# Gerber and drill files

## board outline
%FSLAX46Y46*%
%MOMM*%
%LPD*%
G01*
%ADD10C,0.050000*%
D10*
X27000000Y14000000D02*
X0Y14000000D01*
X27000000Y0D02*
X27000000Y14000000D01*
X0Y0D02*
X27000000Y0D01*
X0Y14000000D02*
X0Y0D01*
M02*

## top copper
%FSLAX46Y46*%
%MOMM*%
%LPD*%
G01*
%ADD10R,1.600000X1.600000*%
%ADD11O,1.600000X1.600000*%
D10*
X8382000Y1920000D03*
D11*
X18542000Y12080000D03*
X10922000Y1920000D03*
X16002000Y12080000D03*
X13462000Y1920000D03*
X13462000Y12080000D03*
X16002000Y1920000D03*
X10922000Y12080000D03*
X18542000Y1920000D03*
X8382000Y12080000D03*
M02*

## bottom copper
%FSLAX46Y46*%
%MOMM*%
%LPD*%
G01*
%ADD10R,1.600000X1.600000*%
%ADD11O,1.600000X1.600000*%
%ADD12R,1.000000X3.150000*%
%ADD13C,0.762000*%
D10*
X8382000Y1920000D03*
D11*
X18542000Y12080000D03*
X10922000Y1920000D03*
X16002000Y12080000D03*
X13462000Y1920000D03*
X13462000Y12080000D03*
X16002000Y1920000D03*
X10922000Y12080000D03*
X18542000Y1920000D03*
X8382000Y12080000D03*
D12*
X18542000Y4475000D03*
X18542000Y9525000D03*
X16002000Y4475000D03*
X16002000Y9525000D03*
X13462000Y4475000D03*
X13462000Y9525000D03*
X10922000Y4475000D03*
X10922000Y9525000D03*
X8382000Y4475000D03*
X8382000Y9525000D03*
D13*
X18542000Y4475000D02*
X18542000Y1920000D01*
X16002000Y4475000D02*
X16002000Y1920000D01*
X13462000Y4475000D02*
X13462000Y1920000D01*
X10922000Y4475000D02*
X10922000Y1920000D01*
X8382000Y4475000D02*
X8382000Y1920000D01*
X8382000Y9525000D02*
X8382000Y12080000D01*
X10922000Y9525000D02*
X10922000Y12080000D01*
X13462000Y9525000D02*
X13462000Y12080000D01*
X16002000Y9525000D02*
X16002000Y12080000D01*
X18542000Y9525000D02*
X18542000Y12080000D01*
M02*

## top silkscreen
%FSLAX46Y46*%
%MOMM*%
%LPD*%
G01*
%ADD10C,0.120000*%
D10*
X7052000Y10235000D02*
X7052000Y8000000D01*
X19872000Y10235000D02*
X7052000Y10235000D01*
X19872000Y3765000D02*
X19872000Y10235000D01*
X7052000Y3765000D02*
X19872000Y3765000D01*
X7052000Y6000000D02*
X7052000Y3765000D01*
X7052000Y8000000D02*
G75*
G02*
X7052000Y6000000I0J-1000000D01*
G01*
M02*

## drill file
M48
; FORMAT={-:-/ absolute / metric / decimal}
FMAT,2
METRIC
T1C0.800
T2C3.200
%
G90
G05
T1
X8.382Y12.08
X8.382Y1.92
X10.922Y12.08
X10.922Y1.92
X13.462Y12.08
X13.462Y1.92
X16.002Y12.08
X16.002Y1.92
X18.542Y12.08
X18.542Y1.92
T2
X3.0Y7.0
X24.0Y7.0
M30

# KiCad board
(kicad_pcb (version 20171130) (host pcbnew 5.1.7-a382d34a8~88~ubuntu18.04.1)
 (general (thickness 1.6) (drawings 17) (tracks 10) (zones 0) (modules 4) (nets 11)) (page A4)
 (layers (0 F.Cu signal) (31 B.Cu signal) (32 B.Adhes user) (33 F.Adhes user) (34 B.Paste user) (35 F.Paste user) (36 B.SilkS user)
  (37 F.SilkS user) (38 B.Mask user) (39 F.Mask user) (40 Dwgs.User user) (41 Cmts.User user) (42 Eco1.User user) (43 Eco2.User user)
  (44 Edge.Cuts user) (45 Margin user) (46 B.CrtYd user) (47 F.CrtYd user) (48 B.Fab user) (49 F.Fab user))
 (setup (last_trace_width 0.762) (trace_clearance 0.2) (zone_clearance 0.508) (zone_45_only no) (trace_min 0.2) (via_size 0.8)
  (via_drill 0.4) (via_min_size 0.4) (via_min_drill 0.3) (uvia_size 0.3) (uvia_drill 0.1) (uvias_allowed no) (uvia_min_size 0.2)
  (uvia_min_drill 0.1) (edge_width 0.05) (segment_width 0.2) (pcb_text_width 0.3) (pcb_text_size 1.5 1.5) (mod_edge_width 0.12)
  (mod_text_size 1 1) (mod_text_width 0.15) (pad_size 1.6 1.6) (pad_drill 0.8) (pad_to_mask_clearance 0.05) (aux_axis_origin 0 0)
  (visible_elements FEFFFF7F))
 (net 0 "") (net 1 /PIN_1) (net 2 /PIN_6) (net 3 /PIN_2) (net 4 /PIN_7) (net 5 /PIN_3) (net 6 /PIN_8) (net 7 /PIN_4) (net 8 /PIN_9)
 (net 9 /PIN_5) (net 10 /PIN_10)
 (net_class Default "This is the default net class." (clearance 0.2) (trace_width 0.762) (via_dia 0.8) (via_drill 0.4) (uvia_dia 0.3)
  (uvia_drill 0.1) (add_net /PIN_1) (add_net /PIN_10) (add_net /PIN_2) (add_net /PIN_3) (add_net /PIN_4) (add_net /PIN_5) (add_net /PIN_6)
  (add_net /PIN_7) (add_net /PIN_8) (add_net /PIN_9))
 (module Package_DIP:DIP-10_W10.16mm (layer F.Cu) (at 8.382 -1.92 90)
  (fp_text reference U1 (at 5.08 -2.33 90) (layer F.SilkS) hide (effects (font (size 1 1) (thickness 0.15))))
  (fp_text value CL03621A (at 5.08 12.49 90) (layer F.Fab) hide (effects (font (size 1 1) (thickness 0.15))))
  (fp_line (start 8.315 -1.33) (end 6.08 -1.33) (layer F.SilkS) (width 0.12))
  (fp_line (start 8.315 11.49) (end 8.315 -1.33) (layer F.SilkS) (width 0.12))
  (fp_line (start 1.845 11.49) (end 8.315 11.49) (layer F.SilkS) (width 0.12))
  (fp_line (start 1.845 -1.33) (end 1.845 11.49) (layer F.SilkS) (width 0.12))
  (fp_line (start 4.08 -1.33) (end 1.845 -1.33) (layer F.SilkS) (width 0.12))
  (fp_arc (start 5.08 -1.33) (end 4.08 -1.33) (angle -180) (layer F.SilkS) (width 0.12))
  (pad 1 thru_hole rect (at 0 0 90) (size 1.6 1.6) (drill 0.8) (layers *.Cu *.Mask) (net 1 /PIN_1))
  (pad 6 thru_hole oval (at 10.16 10.16 90) (size 1.6 1.6) (drill 0.8) (layers *.Cu *.Mask) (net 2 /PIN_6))
  (pad 2 thru_hole oval (at 0 2.54 90) (size 1.6 1.6) (drill 0.8) (layers *.Cu *.Mask) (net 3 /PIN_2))
  (pad 7 thru_hole oval (at 10.16 7.62 90) (size 1.6 1.6) (drill 0.8) (layers *.Cu *.Mask) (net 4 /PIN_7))
  (pad 3 thru_hole oval (at 0 5.08 90) (size 1.6 1.6) (drill 0.8) (layers *.Cu *.Mask) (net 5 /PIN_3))
  (pad 8 thru_hole oval (at 10.16 5.08 90) (size 1.6 1.6) (drill 0.8) (layers *.Cu *.Mask) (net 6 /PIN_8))
  (pad 4 thru_hole oval (at 0 7.62 90) (size 1.6 1.6) (drill 0.8) (layers *.Cu *.Mask) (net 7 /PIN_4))
  (pad 9 thru_hole oval (at 10.16 2.54 90) (size 1.6 1.6) (drill 0.8) (layers *.Cu *.Mask) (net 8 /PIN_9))
  (pad 5 thru_hole oval (at 0 10.16 90) (size 1.6 1.6) (drill 0.8) (layers *.Cu *.Mask) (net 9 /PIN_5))
  (pad 10 thru_hole oval (at 10.16 0 90) (size 1.6 1.6) (drill 0.8) (layers *.Cu *.Mask) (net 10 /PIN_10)))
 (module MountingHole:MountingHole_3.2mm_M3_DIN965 (layer F.Cu) (at 24 -7)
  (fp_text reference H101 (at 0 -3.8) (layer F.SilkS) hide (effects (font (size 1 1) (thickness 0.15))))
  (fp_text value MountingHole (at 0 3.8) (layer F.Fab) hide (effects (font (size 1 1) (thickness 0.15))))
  (pad 1 np_thru_hole circle (at 0 0) (size 3.2 3.2) (drill 3.2) (layers *.Cu *.Mask)))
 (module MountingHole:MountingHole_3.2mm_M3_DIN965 (layer F.Cu) (at 3 -7)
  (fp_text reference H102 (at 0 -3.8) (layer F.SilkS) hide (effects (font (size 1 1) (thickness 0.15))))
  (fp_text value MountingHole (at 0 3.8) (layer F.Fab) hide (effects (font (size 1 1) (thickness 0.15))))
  (pad 1 np_thru_hole circle (at 0 0) (size 3.2 3.2) (drill 3.2) (layers *.Cu *.Mask)))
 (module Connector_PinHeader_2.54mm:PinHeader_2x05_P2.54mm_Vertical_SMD (layer B.Cu) (at 13.462 -7 90)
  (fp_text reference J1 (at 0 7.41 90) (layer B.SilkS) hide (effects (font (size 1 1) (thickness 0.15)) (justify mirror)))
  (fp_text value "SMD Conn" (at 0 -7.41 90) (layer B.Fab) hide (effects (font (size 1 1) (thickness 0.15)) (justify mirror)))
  (pad 1 smd rect (at -2.525 5.08 90) (size 3.15 1) (layers B.Cu B.Paste B.Mask) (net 9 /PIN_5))
  (pad 2 smd rect (at 2.525 5.08 90) (size 3.15 1) (layers B.Cu B.Paste B.Mask) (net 2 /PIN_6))
  (pad 3 smd rect (at -2.525 2.54 90) (size 3.15 1) (layers B.Cu B.Paste B.Mask) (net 7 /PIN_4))
  (pad 4 smd rect (at 2.525 2.54 90) (size 3.15 1) (layers B.Cu B.Paste B.Mask) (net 4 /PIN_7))
  (pad 5 smd rect (at -2.525 0 90) (size 3.15 1) (layers B.Cu B.Paste B.Mask) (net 5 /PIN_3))
  (pad 6 smd rect (at 2.525 0 90) (size 3.15 1) (layers B.Cu B.Paste B.Mask) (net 6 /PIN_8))
  (pad 7 smd rect (at -2.525 -2.54 90) (size 3.15 1) (layers B.Cu B.Paste B.Mask) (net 3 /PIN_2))
  (pad 8 smd rect (at 2.525 -2.54 90) (size 3.15 1) (layers B.Cu B.Paste B.Mask) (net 8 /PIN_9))
  (pad 9 smd rect (at -2.525 -5.08 90) (size 3.15 1) (layers B.Cu B.Paste B.Mask) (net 1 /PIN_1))
  (pad 10 smd rect (at 2.525 -5.08 90) (size 3.15 1) (layers B.Cu B.Paste B.Mask) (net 10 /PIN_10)))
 (gr_line (start 27 -14) (end 0 -14) (layer Edge.Cuts) (width 0.05))
 (gr_line (start 27 0) (end 27 -14) (layer Edge.Cuts) (width 0.05))
 (gr_line (start 0 0) (end 27 0) (layer Edge.Cuts) (width 0.05))
 (gr_line (start 0 -14) (end 0 0) (layer Edge.Cuts) (width 0.05))
 (segment (start 18.542 -4.475) (end 18.542 -1.92) (width 0.762) (layer B.Cu) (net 9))
 (segment (start 16.002 -4.475) (end 16.002 -1.92) (width 0.762) (layer B.Cu) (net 7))
 (segment (start 13.462 -4.475) (end 13.462 -1.92) (width 0.762) (layer B.Cu) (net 5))
 (segment (start 10.922 -4.475) (end 10.922 -1.92) (width 0.762) (layer B.Cu) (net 3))
 (segment (start 8.382 -4.475) (end 8.382 -1.92) (width 0.762) (layer B.Cu) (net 1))
 (segment (start 8.382 -9.525) (end 8.382 -12.08) (width 0.762) (layer B.Cu) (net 10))
 (segment (start 10.922 -9.525) (end 10.922 -12.08) (width 0.762) (layer B.Cu) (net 8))
 (segment (start 13.462 -9.525) (end 13.462 -12.08) (width 0.762) (layer B.Cu) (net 6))
 (segment (start 16.002 -9.525) (end 16.002 -12.08) (width 0.762) (layer B.Cu) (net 4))
 (segment (start 18.542 -9.525) (end 18.542 -12.08) (width 0.762) (layer B.Cu) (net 2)))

